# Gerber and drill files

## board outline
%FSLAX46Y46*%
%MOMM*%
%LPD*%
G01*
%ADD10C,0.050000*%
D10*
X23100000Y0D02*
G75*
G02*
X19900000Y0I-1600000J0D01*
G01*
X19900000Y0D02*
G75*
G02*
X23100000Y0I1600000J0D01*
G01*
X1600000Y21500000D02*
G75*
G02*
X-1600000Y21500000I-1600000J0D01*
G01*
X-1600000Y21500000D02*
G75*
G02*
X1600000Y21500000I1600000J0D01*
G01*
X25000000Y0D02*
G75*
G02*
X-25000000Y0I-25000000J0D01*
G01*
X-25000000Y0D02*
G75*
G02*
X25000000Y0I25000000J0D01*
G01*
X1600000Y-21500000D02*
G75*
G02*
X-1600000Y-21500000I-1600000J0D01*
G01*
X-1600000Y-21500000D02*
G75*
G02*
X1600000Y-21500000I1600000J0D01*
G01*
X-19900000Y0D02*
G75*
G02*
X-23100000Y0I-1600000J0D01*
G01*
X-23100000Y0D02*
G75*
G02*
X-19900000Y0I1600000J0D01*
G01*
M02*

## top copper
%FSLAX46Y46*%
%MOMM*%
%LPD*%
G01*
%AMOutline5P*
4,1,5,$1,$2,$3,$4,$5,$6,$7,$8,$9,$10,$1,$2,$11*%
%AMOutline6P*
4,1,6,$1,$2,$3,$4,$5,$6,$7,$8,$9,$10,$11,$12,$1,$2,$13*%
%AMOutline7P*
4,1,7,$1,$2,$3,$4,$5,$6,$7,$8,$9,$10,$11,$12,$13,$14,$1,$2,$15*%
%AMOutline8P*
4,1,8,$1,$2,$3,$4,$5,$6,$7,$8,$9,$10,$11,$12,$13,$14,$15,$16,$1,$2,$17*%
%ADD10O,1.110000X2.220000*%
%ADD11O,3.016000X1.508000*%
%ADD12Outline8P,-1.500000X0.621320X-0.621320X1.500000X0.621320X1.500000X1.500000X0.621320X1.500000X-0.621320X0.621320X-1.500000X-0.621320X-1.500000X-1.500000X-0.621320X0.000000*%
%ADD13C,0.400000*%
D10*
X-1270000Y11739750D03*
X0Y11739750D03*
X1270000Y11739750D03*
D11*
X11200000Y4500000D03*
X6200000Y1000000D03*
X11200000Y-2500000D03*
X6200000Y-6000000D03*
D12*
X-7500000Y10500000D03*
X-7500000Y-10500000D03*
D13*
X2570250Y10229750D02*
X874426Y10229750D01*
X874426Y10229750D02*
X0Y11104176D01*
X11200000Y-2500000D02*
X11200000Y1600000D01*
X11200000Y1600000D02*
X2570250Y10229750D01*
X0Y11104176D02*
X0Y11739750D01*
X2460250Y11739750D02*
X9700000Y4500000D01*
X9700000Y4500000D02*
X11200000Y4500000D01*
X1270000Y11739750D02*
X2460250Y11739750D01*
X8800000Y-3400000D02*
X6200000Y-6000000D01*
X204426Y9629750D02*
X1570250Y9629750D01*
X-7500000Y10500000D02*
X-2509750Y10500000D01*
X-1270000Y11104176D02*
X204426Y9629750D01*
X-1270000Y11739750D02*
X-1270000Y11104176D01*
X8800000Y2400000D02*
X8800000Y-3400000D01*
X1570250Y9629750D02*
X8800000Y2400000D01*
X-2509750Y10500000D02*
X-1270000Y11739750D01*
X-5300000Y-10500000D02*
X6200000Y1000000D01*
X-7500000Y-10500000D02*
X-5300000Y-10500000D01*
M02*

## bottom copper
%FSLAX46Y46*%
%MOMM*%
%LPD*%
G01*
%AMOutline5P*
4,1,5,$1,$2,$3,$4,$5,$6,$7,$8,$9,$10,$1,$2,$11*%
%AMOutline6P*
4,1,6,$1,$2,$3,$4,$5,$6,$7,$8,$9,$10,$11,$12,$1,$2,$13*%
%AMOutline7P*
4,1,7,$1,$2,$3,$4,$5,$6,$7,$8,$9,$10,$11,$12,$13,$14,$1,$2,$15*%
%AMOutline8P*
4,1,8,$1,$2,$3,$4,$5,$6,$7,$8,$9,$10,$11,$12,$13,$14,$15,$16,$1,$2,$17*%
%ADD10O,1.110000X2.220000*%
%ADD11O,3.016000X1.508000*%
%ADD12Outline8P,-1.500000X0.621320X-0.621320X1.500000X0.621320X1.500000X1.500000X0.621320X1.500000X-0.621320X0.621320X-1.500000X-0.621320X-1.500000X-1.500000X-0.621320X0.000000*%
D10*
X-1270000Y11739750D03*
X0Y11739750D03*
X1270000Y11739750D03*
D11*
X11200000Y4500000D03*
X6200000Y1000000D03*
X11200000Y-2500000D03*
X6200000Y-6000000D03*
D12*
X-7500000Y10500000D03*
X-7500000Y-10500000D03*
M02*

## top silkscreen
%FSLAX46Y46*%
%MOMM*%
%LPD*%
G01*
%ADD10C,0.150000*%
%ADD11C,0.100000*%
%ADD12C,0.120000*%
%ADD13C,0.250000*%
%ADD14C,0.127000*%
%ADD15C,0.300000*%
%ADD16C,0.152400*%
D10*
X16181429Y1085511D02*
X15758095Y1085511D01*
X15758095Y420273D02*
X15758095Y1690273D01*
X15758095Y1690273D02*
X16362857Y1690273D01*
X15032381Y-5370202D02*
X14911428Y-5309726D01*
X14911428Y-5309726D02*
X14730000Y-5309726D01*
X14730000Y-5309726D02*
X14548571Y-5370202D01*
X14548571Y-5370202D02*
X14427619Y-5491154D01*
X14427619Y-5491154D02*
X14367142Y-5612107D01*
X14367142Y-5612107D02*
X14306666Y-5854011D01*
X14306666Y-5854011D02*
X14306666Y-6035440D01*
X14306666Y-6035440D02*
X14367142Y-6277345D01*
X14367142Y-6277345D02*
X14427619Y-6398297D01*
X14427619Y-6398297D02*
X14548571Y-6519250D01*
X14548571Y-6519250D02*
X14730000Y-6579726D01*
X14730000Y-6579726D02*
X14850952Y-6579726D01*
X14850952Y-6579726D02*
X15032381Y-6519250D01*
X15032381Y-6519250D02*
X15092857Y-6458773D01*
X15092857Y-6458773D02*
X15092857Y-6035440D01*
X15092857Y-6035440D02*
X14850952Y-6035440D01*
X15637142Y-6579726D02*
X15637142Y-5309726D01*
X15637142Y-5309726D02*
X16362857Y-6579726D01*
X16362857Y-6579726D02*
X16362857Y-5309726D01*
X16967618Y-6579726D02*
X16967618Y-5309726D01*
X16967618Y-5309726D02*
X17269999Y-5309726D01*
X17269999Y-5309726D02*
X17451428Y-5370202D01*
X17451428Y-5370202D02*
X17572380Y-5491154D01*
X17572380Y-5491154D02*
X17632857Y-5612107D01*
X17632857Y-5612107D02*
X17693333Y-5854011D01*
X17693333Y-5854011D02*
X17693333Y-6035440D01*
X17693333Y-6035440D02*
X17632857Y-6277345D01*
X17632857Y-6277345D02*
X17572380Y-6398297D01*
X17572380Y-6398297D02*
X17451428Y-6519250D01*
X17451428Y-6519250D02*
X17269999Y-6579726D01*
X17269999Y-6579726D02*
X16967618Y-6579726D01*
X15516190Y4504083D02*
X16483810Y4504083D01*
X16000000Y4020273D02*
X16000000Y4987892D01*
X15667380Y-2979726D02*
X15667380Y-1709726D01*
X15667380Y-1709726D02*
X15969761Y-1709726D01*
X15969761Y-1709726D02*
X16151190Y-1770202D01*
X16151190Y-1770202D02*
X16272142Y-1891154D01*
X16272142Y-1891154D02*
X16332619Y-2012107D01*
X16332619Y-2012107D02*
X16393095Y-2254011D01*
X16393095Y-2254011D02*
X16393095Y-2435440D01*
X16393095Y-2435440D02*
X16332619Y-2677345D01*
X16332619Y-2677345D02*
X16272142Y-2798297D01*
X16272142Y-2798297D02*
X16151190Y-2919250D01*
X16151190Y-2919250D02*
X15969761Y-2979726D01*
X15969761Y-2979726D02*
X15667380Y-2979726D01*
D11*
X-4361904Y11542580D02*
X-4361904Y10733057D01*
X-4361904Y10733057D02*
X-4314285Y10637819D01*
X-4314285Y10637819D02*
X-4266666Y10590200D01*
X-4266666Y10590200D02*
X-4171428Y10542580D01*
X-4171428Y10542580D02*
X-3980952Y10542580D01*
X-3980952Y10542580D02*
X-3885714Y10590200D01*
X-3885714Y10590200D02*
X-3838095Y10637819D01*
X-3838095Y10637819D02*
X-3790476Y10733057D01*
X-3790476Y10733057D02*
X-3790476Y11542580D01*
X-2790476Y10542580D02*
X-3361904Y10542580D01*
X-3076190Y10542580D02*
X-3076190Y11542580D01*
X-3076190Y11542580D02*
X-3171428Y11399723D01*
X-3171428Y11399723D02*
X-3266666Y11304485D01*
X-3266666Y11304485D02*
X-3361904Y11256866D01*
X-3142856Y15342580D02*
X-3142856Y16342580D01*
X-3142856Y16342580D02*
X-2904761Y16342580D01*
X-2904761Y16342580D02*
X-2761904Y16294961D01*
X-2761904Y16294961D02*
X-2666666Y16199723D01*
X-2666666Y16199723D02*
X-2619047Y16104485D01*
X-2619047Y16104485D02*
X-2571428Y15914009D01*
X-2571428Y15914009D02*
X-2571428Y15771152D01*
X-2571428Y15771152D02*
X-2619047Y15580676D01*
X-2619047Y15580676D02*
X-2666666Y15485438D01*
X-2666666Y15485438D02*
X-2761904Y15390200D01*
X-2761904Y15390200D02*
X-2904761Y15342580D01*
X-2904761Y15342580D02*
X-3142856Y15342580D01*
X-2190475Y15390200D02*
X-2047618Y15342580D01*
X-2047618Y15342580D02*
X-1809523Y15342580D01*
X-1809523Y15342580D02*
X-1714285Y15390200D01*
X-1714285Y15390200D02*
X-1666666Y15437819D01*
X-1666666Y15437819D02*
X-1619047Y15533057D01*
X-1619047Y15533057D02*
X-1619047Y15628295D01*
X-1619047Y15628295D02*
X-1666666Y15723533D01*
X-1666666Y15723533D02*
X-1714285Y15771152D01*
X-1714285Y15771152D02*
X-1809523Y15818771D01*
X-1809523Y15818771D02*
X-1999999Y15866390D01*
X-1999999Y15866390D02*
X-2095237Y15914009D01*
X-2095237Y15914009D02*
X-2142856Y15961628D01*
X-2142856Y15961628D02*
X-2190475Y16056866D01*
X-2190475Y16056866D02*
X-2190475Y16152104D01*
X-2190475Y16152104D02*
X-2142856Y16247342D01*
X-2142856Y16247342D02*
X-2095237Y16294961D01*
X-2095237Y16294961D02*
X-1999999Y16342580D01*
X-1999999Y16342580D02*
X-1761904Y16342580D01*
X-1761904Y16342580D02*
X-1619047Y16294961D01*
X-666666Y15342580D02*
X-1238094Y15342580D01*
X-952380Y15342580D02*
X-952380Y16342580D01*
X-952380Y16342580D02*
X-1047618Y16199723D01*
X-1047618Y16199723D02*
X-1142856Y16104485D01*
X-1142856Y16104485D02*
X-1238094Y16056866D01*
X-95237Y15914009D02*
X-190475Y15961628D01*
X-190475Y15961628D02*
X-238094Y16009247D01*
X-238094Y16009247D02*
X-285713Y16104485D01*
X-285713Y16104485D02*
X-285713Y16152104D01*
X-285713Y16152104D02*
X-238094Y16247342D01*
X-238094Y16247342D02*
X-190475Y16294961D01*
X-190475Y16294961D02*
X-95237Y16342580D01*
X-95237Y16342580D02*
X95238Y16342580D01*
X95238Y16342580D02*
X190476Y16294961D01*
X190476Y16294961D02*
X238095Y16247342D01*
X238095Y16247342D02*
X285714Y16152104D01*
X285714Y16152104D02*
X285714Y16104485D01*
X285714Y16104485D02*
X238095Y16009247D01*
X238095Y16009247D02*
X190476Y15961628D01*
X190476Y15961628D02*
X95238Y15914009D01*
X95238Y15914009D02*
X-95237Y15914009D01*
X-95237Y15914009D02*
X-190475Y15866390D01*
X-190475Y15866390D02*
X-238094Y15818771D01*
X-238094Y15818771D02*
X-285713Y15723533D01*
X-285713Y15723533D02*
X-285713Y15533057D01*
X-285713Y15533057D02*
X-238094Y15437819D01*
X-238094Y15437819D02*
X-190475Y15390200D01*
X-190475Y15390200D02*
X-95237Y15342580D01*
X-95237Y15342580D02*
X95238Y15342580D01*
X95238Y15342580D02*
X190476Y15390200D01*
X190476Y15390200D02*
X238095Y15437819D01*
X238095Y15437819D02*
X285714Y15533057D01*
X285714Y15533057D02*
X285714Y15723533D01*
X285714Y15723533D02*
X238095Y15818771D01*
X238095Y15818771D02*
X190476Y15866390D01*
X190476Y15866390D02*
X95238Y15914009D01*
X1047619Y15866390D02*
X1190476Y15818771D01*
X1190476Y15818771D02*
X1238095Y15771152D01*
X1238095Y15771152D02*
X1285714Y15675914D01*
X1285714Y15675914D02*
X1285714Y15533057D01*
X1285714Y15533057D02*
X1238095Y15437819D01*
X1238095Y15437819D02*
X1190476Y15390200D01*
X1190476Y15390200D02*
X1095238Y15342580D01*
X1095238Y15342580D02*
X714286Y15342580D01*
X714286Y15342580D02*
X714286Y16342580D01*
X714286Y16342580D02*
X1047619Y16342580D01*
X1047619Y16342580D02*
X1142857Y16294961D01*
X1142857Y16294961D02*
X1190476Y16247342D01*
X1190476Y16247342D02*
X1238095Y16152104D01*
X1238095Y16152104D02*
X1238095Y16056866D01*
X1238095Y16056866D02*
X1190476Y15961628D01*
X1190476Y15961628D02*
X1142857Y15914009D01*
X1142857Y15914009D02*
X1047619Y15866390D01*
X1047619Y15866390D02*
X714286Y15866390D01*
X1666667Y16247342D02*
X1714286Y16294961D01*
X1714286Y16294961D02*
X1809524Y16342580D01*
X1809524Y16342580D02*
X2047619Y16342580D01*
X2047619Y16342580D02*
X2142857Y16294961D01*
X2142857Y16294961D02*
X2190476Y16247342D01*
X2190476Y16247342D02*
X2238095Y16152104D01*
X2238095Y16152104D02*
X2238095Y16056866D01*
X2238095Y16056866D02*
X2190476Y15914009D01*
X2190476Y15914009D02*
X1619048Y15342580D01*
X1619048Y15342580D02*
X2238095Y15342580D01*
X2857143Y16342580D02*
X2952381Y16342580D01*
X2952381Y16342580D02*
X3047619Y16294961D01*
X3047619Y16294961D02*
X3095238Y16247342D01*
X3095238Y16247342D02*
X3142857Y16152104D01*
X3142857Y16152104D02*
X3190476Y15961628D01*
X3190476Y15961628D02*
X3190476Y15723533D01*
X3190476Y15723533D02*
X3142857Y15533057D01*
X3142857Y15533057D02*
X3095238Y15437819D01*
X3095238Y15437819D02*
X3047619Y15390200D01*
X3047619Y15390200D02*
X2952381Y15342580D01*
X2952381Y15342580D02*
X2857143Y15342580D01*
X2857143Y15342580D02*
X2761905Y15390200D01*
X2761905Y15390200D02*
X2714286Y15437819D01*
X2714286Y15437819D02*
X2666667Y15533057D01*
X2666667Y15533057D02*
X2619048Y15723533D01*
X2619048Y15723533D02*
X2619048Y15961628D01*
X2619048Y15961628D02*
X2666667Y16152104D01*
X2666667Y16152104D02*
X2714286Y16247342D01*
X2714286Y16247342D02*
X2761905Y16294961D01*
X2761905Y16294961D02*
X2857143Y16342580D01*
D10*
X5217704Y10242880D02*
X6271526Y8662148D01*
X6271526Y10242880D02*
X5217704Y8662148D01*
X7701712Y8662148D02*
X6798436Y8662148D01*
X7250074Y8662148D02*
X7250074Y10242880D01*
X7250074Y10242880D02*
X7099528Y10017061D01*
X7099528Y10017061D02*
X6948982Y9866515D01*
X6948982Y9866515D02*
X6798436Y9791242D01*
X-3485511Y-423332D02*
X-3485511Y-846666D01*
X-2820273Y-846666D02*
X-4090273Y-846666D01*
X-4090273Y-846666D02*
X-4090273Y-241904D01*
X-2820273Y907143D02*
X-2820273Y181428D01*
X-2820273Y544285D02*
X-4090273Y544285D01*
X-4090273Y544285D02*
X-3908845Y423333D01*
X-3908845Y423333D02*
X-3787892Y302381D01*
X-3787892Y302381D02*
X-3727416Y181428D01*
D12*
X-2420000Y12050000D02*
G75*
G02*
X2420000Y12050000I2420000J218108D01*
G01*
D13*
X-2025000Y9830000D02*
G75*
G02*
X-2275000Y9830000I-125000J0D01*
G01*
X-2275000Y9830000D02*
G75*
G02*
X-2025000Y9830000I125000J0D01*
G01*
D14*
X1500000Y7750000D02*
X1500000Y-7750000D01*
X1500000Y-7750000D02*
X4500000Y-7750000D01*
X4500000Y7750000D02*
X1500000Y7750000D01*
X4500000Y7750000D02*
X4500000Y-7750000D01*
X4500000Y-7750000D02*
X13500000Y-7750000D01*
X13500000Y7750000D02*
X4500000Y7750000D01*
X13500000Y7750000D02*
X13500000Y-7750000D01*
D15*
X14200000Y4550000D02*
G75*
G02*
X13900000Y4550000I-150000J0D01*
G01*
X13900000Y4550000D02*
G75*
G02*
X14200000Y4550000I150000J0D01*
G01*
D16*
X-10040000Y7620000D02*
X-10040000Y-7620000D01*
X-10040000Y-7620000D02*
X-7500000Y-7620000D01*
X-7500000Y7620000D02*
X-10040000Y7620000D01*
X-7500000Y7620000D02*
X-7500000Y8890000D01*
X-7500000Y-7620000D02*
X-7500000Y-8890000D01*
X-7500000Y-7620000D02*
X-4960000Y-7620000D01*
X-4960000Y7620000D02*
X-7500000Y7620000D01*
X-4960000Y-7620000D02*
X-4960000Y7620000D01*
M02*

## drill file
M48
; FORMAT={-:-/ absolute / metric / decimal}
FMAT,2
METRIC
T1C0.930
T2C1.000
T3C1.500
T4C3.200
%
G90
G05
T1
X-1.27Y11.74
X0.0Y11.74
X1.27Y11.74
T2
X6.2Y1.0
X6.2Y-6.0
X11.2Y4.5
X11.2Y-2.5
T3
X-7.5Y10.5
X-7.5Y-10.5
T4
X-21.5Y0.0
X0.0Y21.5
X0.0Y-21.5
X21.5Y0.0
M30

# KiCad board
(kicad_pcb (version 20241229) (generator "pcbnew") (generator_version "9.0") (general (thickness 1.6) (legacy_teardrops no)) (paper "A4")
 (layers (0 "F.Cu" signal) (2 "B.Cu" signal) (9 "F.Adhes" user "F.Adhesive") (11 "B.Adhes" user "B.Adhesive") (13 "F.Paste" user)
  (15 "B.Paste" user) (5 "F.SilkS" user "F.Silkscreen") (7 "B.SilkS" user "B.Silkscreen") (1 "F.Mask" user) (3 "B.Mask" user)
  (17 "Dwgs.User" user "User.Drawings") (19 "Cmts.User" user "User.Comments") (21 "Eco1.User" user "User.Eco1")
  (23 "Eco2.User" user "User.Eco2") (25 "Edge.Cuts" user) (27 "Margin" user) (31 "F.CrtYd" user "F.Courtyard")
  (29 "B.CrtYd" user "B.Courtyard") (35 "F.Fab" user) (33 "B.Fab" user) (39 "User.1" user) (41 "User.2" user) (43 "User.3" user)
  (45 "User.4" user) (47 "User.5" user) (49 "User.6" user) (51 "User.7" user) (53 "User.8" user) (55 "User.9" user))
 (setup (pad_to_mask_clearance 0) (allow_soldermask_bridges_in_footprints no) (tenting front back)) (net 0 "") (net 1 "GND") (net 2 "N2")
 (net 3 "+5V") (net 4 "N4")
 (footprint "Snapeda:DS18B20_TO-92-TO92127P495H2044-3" (layer "F.Cu") (at 0 -12.5)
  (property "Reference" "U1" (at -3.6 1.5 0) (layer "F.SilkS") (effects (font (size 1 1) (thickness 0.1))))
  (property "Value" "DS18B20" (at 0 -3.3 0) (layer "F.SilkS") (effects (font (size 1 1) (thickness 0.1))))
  (fp_arc (start -2.42 0.45) (mid 0 -2.197917) (end 2.42 0.45) (stroke (width 0.12) (type solid)) (layer "F.SilkS"))
  (fp_circle (center -2.15 2.67) (end -2.025 2.67) (stroke (width 0.25) (type solid)) (fill no) (layer "F.SilkS"))
  (pad "1" thru_hole oval (at -1.27 0.76025) (size 1.11 2.22) (drill 0.93) (layers "*.Cu" "*.Mask") (remove_unused_layers no) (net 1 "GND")
   (solder_mask_margin 0.102))
  (pad "2" thru_hole oval (at 0 0.76025) (size 1.11 2.22) (drill 0.93) (layers "*.Cu" "*.Mask") (remove_unused_layers no) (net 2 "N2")
   (solder_mask_margin 0.102))
  (pad "3" thru_hole oval (at 1.27 0.76025) (size 1.11 2.22) (drill 0.93) (layers "*.Cu" "*.Mask") (remove_unused_layers no) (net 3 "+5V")
   (solder_mask_margin 0.102)))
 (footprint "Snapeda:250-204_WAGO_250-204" (layer "F.Cu") (at 7.5 0)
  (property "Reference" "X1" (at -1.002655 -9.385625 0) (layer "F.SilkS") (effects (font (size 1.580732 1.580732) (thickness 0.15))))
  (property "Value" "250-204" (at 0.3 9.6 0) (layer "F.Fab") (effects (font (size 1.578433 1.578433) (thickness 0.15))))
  (fp_line (start -6 -7.75) (end -6 7.75) (stroke (width 0.127) (type solid)) (layer "F.SilkS"))
  (fp_line (start -6 7.75) (end -3 7.75) (stroke (width 0.127) (type solid)) (layer "F.SilkS"))
  (fp_line (start -3 -7.75) (end -6 -7.75) (stroke (width 0.127) (type solid)) (layer "F.SilkS"))
  (fp_line (start -3 -7.75) (end -3 7.75) (stroke (width 0.127) (type solid)) (layer "F.SilkS"))
  (fp_line (start -3 7.75) (end 6 7.75) (stroke (width 0.127) (type solid)) (layer "F.SilkS"))
  (fp_line (start 6 -7.75) (end -3 -7.75) (stroke (width 0.127) (type solid)) (layer "F.SilkS"))
  (fp_line (start 6 -7.75) (end 6 7.75) (stroke (width 0.127) (type solid)) (layer "F.SilkS"))
  (fp_circle (center 6.55 -4.55) (end 6.7 -4.55) (stroke (width 0.3) (type solid)) (fill no) (layer "F.SilkS"))
  (pad "P1" thru_hole oval (at 3.7 -4.5) (size 3.016 1.508) (drill 1) (layers "*.Cu" "*.Mask") (remove_unused_layers no) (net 3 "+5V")
   (solder_mask_margin 0.102))
  (pad "P2" thru_hole oval (at -1.3 -1) (size 3.016 1.508) (drill 1) (layers "*.Cu" "*.Mask") (remove_unused_layers no) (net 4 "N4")
   (solder_mask_margin 0.102))
  (pad "P3" thru_hole oval (at 3.7 2.5) (size 3.016 1.508) (drill 1) (layers "*.Cu" "*.Mask") (remove_unused_layers no) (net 2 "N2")
   (solder_mask_margin 0.102))
  (pad "P4" thru_hole oval (at -1.3 6) (size 3.016 1.508) (drill 1) (layers "*.Cu" "*.Mask") (remove_unused_layers no) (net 1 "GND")
   (solder_mask_margin 0.102)))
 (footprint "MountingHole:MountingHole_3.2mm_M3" (layer "F.Cu") (at 0 -21.5)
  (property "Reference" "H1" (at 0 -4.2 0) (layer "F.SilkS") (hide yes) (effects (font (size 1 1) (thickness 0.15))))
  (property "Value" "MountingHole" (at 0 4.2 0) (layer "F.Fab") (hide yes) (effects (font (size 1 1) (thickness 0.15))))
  (pad "" np_thru_hole circle (at 0 0) (size 3.2 3.2) (drill 3.2) (layers "*.Cu" "*.Mask")))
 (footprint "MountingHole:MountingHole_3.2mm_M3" (layer "F.Cu") (at -21.5 0)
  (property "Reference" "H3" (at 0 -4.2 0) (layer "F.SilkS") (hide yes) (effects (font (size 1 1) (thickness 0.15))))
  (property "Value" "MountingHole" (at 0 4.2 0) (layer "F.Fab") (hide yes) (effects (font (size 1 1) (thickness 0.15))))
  (pad "" np_thru_hole circle (at 0 0) (size 3.2 3.2) (drill 3.2) (layers "*.Cu" "*.Mask")))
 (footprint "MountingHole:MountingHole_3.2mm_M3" (layer "F.Cu") (at 21.5 0)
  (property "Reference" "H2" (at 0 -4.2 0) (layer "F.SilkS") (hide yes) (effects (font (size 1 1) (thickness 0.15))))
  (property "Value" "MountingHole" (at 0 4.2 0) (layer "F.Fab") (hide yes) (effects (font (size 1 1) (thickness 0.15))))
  (pad "" np_thru_hole circle (at 0 0) (size 3.2 3.2) (drill 3.2) (layers "*.Cu" "*.Mask")))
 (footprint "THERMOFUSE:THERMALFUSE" (layer "F.Cu") (at -7.5 0)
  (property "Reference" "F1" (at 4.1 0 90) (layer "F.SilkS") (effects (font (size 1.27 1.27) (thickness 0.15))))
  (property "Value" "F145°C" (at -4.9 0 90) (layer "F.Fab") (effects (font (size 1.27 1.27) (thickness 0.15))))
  (fp_line (start -2.54 -7.62) (end -2.54 7.62) (stroke (width 0.1524) (type solid)) (layer "F.SilkS"))
  (fp_line (start -2.54 7.62) (end 0 7.62) (stroke (width 0.1524) (type solid)) (layer "F.SilkS"))
  (fp_line (start 0 -7.62) (end -2.54 -7.62) (stroke (width 0.1524) (type solid)) (layer "F.SilkS"))
  (fp_line (start 0 -7.62) (end 0 -8.89) (stroke (width 0.1524) (type solid)) (layer "F.SilkS"))
  (fp_line (start 0 7.62) (end 0 8.89) (stroke (width 0.1524) (type solid)) (layer "F.SilkS"))
  (fp_line (start 0 7.62) (end 2.54 7.62) (stroke (width 0.1524) (type solid)) (layer "F.SilkS"))
  (fp_line (start 2.54 -7.62) (end 0 -7.62) (stroke (width 0.1524) (type solid)) (layer "F.SilkS"))
  (fp_line (start 2.54 7.62) (end 2.54 -7.62) (stroke (width 0.1524) (type solid)) (layer "F.SilkS"))
  (pad "1" thru_hole roundrect (at 0 -10.5) (size 3 3) (drill 1.5) (layers "*.Cu" "*.Mask") (remove_unused_layers no)
   (roundrect_rratio 0.25) (chamfer_ratio 0.2928932188) (chamfer top_left top_right bottom_left bottom_right) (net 1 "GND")
   (solder_mask_margin 0.1016) (thermal_bridge_angle 0))
  (pad "2" thru_hole roundrect (at 0 10.5) (size 3 3) (drill 1.5) (layers "*.Cu" "*.Mask") (remove_unused_layers no) (roundrect_rratio 0.25)
   (chamfer_ratio 0.2928932188) (chamfer top_left top_right bottom_left bottom_right) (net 4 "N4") (solder_mask_margin 0.1016)
   (thermal_bridge_angle 0)))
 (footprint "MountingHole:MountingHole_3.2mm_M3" (layer "F.Cu") (at 0 21.5)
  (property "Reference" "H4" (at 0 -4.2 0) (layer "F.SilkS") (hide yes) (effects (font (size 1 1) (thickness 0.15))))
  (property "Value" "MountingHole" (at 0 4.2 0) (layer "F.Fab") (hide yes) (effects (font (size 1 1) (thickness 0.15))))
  (pad "" np_thru_hole circle (at 0 0) (size 3.2 3.2) (drill 3.2) (layers "*.Cu" "*.Mask")))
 (gr_circle (center 21.5 0) (end 23.1 0) (stroke (width 0.05) (type default)) (fill no) (layer "Edge.Cuts"))
 (gr_circle (center 0 -21.5) (end 1.6 -21.5) (stroke (width 0.05) (type default)) (fill no) (layer "Edge.Cuts"))
 (gr_circle (center 0 0) (end 25 0) (stroke (width 0.05) (type default)) (fill no) (layer "Edge.Cuts"))
 (gr_circle (center 0 21.5) (end 1.6 21.5) (stroke (width 0.05) (type default)) (fill no) (layer "Edge.Cuts"))
 (gr_circle (center -21.5 0) (end -19.9 0) (stroke (width 0.05) (type default)) (fill no) (layer "Edge.Cuts"))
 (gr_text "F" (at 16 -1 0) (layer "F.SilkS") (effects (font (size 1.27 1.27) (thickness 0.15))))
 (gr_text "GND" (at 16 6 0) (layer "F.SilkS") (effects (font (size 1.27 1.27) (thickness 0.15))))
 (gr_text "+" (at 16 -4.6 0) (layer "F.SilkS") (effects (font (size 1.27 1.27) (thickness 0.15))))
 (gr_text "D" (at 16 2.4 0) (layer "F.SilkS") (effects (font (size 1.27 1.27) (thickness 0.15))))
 (segment (start 2.57025 -10.22975) (end 0.874426 -10.22975) (width 0.4) (layer "F.Cu") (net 2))
 (segment (start 0.874426 -10.22975) (end 0 -11.104176) (width 0.4) (layer "F.Cu") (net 2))
 (segment (start 11.2 2.5) (end 11.2 -1.6) (width 0.4) (layer "F.Cu") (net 2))
 (segment (start 11.2 -1.6) (end 2.57025 -10.22975) (width 0.4) (layer "F.Cu") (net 2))
 (segment (start 0 -11.104176) (end 0 -11.73975) (width 0.4) (layer "F.Cu") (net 2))
 (segment (start 2.46025 -11.73975) (end 9.7 -4.5) (width 0.4) (layer "F.Cu") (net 3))
 (segment (start 9.7 -4.5) (end 11.2 -4.5) (width 0.4) (layer "F.Cu") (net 3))
 (segment (start 1.27 -11.73975) (end 2.46025 -11.73975) (width 0.4) (layer "F.Cu") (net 3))
 (segment (start 8.8 3.4) (end 6.2 6) (width 0.4) (layer "F.Cu") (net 1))
 (segment (start 0.204426 -9.62975) (end 1.57025 -9.62975) (width 0.4) (layer "F.Cu") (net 1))
 (segment (start -7.5 -10.5) (end -2.50975 -10.5) (width 0.4) (layer "F.Cu") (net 1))
 (segment (start -1.27 -11.104176) (end 0.204426 -9.62975) (width 0.4) (layer "F.Cu") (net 1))
 (segment (start -1.27 -11.73975) (end -1.27 -11.104176) (width 0.4) (layer "F.Cu") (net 1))
 (segment (start 8.8 -2.4) (end 8.8 3.4) (width 0.4) (layer "F.Cu") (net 1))
 (segment (start 1.57025 -9.62975) (end 8.8 -2.4) (width 0.4) (layer "F.Cu") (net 1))
 (segment (start -2.50975 -10.5) (end -1.27 -11.73975) (width 0.4) (layer "F.Cu") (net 1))
 (segment (start -5.3 10.5) (end 6.2 -1) (width 0.4) (layer "F.Cu") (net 4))
 (segment (start -7.5 10.5) (end -5.3 10.5) (width 0.4) (layer "F.Cu") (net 4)))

